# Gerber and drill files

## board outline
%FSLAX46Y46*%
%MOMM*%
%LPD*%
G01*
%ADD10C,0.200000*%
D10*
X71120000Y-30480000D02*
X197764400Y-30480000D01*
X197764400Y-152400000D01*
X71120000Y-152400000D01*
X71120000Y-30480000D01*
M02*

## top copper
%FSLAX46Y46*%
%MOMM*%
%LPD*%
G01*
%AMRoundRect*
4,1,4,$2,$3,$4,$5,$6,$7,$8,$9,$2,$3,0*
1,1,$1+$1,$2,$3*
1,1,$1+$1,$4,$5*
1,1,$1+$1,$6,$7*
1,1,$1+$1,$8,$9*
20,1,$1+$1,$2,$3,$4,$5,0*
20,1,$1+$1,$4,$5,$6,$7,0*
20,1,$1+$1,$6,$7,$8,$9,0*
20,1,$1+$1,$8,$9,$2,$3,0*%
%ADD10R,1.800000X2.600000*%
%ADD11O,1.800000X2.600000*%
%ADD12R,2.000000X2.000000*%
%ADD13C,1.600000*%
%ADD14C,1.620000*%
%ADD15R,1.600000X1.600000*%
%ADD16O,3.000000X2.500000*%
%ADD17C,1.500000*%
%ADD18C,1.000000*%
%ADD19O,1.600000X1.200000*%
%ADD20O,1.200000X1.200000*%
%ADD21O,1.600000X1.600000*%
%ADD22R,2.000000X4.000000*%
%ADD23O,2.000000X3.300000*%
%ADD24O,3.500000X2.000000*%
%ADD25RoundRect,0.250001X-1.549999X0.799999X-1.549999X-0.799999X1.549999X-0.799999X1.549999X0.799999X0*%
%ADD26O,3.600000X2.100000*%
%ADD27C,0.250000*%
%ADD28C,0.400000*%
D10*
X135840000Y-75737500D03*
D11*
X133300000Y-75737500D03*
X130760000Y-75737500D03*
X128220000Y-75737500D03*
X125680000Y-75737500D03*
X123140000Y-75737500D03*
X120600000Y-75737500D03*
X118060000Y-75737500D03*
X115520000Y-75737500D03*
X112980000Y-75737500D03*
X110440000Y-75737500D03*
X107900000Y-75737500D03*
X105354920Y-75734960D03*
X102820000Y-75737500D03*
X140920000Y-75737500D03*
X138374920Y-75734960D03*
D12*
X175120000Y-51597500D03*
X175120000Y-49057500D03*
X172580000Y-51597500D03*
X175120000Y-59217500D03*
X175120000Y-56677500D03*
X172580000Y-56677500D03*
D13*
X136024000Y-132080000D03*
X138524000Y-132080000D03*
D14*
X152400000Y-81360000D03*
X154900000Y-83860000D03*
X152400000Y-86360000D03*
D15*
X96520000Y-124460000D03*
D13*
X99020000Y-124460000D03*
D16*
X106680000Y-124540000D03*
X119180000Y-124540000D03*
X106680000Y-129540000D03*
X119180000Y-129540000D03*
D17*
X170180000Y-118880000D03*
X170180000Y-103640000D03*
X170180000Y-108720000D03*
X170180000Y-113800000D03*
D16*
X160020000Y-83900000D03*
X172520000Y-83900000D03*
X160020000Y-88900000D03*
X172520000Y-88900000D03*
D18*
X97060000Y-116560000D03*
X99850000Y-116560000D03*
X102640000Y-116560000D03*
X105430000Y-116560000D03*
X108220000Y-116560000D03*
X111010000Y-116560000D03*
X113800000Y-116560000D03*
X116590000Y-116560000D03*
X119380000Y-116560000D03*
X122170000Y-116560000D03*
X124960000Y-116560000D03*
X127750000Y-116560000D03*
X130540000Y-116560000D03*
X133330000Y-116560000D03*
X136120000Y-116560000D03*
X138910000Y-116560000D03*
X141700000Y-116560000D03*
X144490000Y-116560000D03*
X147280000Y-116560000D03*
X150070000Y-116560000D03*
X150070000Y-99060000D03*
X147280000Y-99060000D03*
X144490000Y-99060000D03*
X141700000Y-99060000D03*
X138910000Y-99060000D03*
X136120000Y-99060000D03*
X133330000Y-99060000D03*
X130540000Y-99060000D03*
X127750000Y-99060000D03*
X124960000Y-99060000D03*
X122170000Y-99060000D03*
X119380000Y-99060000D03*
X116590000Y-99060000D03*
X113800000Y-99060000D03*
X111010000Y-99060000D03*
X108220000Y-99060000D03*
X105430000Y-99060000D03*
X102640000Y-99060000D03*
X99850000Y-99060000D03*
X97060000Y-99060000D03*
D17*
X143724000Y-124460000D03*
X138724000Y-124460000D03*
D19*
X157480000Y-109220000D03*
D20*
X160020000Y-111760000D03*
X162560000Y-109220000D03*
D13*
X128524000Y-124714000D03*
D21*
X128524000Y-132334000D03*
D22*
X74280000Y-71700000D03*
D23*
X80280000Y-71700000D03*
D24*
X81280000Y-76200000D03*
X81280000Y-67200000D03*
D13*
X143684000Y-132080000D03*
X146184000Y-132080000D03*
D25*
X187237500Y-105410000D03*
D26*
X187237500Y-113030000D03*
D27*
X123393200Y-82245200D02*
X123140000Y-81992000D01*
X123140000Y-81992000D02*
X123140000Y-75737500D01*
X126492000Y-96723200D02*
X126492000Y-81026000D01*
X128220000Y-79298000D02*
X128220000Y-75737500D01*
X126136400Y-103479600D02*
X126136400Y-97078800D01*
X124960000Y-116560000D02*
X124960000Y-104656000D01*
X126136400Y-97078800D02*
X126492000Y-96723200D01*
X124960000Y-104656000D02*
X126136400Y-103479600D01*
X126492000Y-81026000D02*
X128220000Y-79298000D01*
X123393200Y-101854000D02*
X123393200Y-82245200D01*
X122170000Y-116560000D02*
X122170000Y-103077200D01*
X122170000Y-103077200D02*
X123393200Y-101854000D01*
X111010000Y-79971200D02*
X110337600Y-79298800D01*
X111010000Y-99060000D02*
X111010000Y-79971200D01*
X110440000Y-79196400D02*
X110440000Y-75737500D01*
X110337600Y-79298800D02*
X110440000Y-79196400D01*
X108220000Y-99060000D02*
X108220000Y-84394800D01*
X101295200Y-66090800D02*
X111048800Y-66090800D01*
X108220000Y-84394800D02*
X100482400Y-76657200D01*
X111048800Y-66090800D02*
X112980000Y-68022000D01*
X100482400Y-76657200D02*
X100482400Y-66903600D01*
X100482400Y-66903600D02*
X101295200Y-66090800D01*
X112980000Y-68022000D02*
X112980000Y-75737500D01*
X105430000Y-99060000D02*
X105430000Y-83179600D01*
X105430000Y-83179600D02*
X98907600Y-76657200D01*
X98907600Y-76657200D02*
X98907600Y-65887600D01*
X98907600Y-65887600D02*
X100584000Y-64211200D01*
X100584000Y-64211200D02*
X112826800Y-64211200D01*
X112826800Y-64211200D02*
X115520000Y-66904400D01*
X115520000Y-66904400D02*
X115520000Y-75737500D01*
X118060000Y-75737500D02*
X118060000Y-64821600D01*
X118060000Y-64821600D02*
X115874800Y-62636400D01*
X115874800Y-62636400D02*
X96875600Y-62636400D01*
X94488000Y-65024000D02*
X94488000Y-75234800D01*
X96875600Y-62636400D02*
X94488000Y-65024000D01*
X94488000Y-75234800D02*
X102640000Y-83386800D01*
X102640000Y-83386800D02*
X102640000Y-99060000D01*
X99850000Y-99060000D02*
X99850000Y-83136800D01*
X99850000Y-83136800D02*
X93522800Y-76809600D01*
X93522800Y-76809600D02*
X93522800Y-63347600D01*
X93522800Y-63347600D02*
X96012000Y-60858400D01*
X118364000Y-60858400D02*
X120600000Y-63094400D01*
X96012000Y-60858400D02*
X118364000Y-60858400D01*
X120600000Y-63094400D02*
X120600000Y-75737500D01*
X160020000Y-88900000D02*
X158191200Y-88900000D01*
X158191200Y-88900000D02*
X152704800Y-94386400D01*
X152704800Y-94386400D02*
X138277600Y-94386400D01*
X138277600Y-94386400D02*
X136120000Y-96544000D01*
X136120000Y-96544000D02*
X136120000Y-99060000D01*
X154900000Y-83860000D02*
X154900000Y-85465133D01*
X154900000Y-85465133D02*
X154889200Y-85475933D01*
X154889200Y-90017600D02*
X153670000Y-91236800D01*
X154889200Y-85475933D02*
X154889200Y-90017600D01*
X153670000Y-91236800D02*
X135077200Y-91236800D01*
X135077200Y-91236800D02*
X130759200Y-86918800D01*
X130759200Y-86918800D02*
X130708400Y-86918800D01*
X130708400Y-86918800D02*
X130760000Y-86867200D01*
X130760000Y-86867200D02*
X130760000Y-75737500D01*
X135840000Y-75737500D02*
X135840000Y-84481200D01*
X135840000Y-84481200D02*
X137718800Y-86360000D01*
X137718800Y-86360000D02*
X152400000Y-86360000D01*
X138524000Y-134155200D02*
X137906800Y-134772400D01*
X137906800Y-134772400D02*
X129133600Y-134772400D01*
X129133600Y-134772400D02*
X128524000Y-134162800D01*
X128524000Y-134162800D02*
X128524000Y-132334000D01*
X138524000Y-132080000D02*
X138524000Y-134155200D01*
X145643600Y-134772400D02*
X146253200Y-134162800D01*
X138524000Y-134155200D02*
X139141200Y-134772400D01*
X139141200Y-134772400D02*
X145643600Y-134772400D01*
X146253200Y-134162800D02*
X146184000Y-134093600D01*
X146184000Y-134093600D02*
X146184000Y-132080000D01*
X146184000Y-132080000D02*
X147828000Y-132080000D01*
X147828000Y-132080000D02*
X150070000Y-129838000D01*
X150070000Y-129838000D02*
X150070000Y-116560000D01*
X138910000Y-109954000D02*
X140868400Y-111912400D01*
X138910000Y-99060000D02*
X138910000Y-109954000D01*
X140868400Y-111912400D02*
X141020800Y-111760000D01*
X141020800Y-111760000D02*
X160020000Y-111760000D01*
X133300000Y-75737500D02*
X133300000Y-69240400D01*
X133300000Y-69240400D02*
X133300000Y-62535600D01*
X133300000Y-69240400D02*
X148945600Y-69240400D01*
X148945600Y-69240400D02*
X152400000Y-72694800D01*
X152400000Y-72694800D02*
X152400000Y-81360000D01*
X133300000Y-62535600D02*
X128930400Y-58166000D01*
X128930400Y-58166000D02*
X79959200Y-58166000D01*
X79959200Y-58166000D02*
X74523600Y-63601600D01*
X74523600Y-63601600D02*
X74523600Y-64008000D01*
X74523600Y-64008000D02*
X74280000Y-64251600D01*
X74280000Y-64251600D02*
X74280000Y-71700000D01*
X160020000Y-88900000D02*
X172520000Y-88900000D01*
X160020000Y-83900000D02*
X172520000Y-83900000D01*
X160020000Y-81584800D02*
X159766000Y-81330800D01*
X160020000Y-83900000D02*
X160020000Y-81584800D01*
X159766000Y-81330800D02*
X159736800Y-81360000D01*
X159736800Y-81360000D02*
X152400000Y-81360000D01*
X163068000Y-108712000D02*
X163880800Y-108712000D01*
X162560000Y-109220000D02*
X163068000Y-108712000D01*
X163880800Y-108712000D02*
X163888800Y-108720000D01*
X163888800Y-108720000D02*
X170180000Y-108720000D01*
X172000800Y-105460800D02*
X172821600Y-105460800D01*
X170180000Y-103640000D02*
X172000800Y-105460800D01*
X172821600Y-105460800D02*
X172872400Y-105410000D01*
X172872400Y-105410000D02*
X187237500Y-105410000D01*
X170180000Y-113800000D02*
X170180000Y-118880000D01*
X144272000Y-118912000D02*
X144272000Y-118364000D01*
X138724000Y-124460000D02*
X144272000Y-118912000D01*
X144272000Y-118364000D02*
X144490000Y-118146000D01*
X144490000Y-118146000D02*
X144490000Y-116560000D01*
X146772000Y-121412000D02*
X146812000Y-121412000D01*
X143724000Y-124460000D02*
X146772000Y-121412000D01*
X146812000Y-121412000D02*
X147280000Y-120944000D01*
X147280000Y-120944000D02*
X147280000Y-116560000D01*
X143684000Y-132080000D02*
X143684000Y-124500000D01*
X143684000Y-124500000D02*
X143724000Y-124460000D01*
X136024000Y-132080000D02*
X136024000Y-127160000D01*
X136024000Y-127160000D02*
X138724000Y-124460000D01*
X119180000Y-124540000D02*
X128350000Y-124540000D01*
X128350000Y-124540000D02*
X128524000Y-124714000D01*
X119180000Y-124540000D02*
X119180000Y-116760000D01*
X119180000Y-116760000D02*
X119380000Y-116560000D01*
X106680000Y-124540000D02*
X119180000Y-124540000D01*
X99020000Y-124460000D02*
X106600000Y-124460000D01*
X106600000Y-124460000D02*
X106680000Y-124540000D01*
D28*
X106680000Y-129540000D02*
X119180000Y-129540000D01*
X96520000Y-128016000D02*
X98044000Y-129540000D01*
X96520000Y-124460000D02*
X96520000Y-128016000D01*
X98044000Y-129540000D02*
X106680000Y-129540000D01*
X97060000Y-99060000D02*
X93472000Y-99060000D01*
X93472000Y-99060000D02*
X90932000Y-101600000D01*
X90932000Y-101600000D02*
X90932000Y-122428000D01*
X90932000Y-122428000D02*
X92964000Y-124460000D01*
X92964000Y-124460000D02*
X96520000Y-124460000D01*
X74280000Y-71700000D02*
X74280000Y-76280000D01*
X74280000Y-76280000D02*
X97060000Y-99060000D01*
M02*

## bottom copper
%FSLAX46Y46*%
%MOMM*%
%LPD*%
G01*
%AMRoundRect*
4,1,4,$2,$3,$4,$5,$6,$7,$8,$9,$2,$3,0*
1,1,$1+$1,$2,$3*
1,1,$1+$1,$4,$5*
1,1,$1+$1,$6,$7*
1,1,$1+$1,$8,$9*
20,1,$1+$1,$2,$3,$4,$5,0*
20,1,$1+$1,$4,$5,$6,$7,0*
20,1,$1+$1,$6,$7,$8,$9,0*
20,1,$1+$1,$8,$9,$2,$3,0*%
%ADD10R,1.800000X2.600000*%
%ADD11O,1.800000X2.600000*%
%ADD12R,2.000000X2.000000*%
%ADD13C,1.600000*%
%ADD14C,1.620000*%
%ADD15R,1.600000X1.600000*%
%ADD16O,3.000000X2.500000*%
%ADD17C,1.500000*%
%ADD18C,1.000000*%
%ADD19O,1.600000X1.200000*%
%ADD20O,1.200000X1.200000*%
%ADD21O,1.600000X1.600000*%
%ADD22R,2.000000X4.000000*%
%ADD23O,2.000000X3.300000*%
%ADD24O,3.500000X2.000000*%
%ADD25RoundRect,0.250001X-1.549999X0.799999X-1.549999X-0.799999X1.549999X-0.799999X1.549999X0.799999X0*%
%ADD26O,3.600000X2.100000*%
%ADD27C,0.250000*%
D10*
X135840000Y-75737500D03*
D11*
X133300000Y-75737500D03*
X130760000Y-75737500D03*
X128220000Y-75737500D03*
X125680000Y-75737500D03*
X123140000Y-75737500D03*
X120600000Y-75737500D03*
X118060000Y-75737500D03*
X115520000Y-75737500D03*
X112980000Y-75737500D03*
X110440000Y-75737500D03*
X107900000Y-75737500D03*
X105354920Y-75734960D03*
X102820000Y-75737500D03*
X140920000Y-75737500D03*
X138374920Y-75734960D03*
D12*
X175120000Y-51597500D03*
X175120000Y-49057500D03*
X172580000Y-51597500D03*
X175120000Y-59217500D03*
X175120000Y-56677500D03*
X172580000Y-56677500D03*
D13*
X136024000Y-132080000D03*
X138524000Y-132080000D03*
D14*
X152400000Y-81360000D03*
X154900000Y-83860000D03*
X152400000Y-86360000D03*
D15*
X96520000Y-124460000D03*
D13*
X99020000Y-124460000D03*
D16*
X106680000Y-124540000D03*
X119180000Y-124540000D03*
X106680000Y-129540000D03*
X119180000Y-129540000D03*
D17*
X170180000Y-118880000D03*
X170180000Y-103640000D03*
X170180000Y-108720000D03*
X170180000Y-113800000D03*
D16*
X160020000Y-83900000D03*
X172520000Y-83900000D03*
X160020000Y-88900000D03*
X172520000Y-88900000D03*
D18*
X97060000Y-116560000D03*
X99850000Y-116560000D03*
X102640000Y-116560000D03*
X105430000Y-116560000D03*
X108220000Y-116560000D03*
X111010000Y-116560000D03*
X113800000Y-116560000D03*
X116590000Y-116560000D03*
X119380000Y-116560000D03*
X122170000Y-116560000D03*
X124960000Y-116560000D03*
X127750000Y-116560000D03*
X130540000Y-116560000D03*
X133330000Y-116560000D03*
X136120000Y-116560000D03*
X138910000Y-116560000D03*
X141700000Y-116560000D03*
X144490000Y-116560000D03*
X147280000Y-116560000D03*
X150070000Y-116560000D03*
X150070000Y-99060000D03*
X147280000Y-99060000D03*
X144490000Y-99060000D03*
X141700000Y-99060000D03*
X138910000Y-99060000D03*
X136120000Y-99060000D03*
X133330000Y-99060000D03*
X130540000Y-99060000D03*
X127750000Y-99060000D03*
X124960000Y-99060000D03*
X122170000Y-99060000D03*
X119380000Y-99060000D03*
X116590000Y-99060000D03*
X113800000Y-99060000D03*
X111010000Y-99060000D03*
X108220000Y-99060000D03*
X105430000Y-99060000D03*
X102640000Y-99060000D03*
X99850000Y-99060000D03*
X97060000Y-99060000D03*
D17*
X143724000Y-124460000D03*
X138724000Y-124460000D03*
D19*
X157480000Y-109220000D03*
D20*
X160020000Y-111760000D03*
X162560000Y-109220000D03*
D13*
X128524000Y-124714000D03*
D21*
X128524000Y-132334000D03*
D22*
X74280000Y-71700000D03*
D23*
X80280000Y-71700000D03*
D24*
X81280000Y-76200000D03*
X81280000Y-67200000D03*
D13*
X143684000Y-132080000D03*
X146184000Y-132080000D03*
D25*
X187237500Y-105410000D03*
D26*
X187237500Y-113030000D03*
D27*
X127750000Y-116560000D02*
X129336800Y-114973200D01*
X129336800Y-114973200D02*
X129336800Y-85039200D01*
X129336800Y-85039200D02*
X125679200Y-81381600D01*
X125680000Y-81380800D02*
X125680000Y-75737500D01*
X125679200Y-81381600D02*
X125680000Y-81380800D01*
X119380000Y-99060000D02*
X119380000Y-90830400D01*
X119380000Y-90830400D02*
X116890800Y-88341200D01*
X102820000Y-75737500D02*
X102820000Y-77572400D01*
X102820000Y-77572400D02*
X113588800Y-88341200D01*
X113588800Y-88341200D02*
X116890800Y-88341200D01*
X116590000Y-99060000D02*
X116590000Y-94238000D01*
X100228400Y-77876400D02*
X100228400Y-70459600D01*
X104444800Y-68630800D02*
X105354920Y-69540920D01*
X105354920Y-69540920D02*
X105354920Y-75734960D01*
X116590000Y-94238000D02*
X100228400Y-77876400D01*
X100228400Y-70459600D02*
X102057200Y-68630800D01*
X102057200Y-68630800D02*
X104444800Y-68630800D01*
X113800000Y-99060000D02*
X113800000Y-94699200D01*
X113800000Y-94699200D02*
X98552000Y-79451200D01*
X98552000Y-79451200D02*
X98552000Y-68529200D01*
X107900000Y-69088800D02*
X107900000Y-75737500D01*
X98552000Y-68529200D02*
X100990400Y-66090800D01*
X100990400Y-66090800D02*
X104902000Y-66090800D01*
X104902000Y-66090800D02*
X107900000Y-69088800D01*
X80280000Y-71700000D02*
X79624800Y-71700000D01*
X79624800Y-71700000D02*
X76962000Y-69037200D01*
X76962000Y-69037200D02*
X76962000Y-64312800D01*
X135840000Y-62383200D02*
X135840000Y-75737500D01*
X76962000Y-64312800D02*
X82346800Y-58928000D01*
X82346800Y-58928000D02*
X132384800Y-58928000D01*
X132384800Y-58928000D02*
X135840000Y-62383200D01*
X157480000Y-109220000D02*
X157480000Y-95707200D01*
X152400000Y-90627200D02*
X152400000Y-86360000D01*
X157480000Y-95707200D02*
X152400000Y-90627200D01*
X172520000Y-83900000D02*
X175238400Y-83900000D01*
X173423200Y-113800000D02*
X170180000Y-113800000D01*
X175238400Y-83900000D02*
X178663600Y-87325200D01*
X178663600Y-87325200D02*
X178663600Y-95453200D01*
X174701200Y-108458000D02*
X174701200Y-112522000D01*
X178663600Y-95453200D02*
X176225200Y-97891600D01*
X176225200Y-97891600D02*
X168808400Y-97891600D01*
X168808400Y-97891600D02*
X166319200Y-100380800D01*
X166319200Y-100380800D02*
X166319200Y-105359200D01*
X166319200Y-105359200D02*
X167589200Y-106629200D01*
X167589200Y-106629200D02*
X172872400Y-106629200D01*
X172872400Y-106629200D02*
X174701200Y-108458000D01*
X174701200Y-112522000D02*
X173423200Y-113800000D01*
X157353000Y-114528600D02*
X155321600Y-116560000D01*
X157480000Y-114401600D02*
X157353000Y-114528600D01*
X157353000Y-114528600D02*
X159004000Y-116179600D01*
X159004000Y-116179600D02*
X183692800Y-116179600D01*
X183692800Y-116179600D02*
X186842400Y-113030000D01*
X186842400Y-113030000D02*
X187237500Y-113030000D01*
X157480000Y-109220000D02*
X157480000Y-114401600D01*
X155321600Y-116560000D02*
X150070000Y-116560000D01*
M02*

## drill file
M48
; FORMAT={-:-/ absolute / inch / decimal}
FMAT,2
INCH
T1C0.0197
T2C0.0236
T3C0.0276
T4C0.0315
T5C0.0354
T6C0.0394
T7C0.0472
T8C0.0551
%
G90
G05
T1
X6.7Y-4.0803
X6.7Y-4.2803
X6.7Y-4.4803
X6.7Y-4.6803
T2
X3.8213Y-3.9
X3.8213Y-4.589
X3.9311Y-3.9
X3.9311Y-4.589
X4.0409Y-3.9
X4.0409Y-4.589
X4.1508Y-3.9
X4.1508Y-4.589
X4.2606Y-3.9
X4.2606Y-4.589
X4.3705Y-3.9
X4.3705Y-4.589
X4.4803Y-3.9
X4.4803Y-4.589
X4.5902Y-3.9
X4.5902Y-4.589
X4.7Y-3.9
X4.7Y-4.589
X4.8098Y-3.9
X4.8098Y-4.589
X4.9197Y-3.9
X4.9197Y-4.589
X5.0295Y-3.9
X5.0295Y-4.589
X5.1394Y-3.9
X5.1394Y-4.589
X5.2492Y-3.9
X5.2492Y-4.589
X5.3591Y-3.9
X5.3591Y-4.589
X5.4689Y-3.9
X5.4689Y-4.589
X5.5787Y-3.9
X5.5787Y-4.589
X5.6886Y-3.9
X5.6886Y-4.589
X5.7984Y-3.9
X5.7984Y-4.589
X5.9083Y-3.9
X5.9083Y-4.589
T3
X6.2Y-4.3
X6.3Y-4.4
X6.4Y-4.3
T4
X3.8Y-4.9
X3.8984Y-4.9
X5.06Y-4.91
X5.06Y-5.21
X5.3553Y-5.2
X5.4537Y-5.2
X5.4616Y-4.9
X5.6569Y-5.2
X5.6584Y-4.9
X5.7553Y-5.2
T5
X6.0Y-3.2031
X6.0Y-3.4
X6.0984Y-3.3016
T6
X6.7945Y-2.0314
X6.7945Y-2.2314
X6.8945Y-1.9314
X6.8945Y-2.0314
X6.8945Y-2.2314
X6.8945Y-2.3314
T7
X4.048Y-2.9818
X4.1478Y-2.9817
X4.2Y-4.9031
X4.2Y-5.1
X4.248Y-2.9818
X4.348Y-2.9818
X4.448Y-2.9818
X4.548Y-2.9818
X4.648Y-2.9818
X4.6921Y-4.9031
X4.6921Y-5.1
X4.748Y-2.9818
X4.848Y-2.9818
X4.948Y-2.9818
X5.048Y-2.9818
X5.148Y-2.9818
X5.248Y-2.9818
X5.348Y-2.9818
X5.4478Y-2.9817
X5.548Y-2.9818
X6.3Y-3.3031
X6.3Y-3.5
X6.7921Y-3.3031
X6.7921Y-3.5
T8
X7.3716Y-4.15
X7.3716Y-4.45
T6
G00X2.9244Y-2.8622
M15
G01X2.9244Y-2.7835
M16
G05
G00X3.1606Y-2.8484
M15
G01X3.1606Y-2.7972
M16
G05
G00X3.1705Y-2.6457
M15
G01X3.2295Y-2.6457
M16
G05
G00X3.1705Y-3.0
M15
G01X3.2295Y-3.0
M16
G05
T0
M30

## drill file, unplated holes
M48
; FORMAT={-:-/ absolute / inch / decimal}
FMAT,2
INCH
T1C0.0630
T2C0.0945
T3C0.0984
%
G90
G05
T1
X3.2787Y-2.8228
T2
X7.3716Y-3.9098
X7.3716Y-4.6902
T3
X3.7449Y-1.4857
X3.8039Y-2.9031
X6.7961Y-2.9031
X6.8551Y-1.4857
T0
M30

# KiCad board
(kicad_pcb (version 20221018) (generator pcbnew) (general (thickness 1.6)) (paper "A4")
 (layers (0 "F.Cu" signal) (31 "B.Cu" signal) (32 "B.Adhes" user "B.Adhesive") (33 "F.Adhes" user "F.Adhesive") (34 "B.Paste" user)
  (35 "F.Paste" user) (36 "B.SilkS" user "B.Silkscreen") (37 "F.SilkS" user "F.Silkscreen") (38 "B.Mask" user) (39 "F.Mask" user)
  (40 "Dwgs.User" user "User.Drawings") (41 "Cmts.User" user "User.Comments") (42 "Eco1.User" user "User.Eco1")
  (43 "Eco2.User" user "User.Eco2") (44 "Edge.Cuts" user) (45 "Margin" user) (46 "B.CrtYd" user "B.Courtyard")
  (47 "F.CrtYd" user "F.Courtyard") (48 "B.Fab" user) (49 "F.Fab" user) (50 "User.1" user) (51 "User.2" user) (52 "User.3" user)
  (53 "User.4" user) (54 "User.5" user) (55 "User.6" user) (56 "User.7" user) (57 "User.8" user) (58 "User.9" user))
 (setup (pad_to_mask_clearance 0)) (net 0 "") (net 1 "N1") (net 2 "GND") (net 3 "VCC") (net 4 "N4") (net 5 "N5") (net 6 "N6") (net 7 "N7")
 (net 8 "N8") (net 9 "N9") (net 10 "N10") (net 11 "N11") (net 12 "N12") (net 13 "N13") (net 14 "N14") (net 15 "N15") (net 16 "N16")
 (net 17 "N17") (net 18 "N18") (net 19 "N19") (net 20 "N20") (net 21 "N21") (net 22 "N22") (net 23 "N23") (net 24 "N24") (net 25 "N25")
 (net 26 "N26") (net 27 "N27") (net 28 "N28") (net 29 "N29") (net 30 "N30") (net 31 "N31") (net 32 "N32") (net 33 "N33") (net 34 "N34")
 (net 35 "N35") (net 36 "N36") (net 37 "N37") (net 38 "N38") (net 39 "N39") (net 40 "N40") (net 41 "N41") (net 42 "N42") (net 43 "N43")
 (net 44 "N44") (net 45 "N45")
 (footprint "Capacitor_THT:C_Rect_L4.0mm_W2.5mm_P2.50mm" (layer "F.Cu") (at 136.024 132.08)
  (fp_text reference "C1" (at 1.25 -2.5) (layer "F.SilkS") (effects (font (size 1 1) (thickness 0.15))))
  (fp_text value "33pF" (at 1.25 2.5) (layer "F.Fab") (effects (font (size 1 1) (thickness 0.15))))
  (pad "1" thru_hole circle (at 0 0) (size 1.6 1.6) (drill 0.8) (layers "*.Cu" "*.Mask") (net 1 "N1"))
  (pad "2" thru_hole circle (at 2.5 0) (size 1.6 1.6) (drill 0.8) (layers "*.Cu" "*.Mask") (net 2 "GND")))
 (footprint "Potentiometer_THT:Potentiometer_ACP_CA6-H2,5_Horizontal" (layer "F.Cu") (at 152.4 81.36)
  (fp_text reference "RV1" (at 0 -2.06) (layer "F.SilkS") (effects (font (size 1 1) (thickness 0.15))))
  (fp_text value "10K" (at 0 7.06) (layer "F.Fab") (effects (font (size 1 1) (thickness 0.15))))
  (pad "1" thru_hole circle (at 0 0) (size 1.62 1.62) (drill 0.9) (layers "*.Cu" "*.Mask") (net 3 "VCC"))
  (pad "2" thru_hole circle (at 2.5 2.5) (size 1.62 1.62) (drill 0.9) (layers "*.Cu" "*.Mask") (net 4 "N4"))
  (pad "3" thru_hole circle (at 0 5) (size 1.62 1.62) (drill 0.9) (layers "*.Cu" "*.Mask") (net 2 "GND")))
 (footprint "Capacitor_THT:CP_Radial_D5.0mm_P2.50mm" (layer "F.Cu") (at 96.52 124.46)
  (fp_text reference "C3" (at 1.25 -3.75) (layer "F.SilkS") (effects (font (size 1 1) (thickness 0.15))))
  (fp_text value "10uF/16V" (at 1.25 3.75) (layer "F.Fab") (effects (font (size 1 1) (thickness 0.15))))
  (pad "1" thru_hole rect (at 0 0) (size 1.6 1.6) (drill 0.8) (layers "*.Cu" "*.Mask") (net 3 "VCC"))
  (pad "2" thru_hole circle (at 2.5 0) (size 1.6 1.6) (drill 0.8) (layers "*.Cu" "*.Mask") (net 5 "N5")))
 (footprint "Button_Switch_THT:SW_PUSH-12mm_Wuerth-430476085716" (layer "F.Cu") (at 106.68 124.54)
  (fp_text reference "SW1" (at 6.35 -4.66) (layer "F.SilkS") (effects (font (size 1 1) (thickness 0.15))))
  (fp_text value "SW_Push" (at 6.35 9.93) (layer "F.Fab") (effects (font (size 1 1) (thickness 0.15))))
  (pad "1" thru_hole oval (at 0 0) (size 3 2.5) (drill 1.2) (layers "*.Cu" "*.Mask") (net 5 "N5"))
  (pad "1" thru_hole oval (at 12.5 0) (size 3 2.5) (drill 1.2) (layers "*.Cu" "*.Mask") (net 5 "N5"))
  (pad "2" thru_hole oval (at 0 5) (size 3 2.5) (drill 1.2) (layers "*.Cu" "*.Mask") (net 3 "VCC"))
  (pad "2" thru_hole oval (at 12.5 5) (size 3 2.5) (drill 1.2) (layers "*.Cu" "*.Mask") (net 3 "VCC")))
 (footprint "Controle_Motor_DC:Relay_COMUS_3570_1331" (layer "F.Cu") (at 170.16 111.74 90)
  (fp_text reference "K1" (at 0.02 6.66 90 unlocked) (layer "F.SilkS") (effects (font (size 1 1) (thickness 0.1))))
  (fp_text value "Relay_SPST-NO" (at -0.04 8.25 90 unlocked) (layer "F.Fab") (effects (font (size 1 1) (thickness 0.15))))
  (pad "13" thru_hole circle (at -7.14 0.02 90) (size 1.5 1.5) (drill 0.5) (layers "*.Cu" "*.Mask") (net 3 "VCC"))
  (pad "14" thru_hole circle (at 8.1 0.02 90) (size 1.5 1.5) (drill 0.5) (layers "*.Cu" "*.Mask") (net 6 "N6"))
  (pad "A1" thru_hole circle (at 3.02 0.02 90) (size 1.5 1.5) (drill 0.5) (layers "*.Cu" "*.Mask") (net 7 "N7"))
  (pad "A2" thru_hole circle (at -2.06 0.02 90) (size 1.5 1.5) (drill 0.5) (layers "*.Cu" "*.Mask") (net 3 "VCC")))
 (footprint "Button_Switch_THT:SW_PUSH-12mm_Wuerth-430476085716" (layer "F.Cu") (at 160.02 83.9)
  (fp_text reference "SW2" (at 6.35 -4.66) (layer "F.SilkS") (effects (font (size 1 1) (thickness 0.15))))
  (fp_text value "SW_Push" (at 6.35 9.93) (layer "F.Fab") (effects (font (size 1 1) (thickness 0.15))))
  (pad "1" thru_hole oval (at 0 0) (size 3 2.5) (drill 1.2) (layers "*.Cu" "*.Mask") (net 3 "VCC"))
  (pad "1" thru_hole oval (at 12.5 0) (size 3 2.5) (drill 1.2) (layers "*.Cu" "*.Mask") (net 3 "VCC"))
  (pad "2" thru_hole oval (at 0 5) (size 3 2.5) (drill 1.2) (layers "*.Cu" "*.Mask") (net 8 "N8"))
  (pad "2" thru_hole oval (at 12.5 5) (size 3 2.5) (drill 1.2) (layers "*.Cu" "*.Mask") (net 8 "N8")))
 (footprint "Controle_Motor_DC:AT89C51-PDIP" (layer "F.Cu") (at 97.06 116.56)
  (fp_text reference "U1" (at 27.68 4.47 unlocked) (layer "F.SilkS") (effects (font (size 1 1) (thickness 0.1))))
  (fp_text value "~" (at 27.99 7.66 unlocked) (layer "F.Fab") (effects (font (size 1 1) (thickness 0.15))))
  (pad "1" thru_hole circle (at 0 0) (size 1 1) (drill 0.6) (layers "*.Cu" "*.Mask") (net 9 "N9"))
  (pad "2" thru_hole circle (at 2.79 0) (size 1 1) (drill 0.6) (layers "*.Cu" "*.Mask") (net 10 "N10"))
  (pad "3" thru_hole circle (at 5.58 0) (size 1 1) (drill 0.6) (layers "*.Cu" "*.Mask") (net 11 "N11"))
  (pad "4" thru_hole circle (at 8.37 0) (size 1 1) (drill 0.6) (layers "*.Cu" "*.Mask") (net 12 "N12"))
  (pad "5" thru_hole circle (at 11.16 0) (size 1 1) (drill 0.6) (layers "*.Cu" "*.Mask") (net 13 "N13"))
  (pad "6" thru_hole circle (at 13.95 0) (size 1 1) (drill 0.6) (layers "*.Cu" "*.Mask") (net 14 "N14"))
  (pad "7" thru_hole circle (at 16.74 0) (size 1 1) (drill 0.6) (layers "*.Cu" "*.Mask") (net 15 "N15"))
  (pad "8" thru_hole circle (at 19.53 0) (size 1 1) (drill 0.6) (layers "*.Cu" "*.Mask") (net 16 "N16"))
  (pad "9" thru_hole circle (at 22.32 0) (size 1 1) (drill 0.6) (layers "*.Cu" "*.Mask") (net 5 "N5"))
  (pad "10" thru_hole circle (at 25.11 0) (size 1 1) (drill 0.6) (layers "*.Cu" "*.Mask") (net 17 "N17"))
  (pad "11" thru_hole circle (at 27.9 0) (size 1 1) (drill 0.6) (layers "*.Cu" "*.Mask") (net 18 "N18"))
  (pad "12" thru_hole circle (at 30.69 0) (size 1 1) (drill 0.6) (layers "*.Cu" "*.Mask") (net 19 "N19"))
  (pad "13" thru_hole circle (at 33.48 0) (size 1 1) (drill 0.6) (layers "*.Cu" "*.Mask") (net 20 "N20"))
  (pad "14" thru_hole circle (at 36.27 0) (size 1 1) (drill 0.6) (layers "*.Cu" "*.Mask") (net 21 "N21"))
  (pad "15" thru_hole circle (at 39.06 0) (size 1 1) (drill 0.6) (layers "*.Cu" "*.Mask") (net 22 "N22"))
  (pad "16" thru_hole circle (at 41.85 0) (size 1 1) (drill 0.6) (layers "*.Cu" "*.Mask") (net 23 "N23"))
  (pad "17" thru_hole circle (at 44.64 0) (size 1 1) (drill 0.6) (layers "*.Cu" "*.Mask") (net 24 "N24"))
  (pad "18" thru_hole circle (at 47.43 0) (size 1 1) (drill 0.6) (layers "*.Cu" "*.Mask") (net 1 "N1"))
  (pad "19" thru_hole circle (at 50.22 0) (size 1 1) (drill 0.6) (layers "*.Cu" "*.Mask") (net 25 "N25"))
  (pad "20" thru_hole circle (at 53.01 0) (size 1 1) (drill 0.6) (layers "*.Cu" "*.Mask") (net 2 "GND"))
  (pad "21" thru_hole circle (at 53.01 -17.5) (size 1 1) (drill 0.6) (layers "*.Cu" "*.Mask") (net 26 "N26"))
  (pad "22" thru_hole circle (at 50.22 -17.5) (size 1 1) (drill 0.6) (layers "*.Cu" "*.Mask") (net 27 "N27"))
  (pad "23" thru_hole circle (at 47.43 -17.5) (size 1 1) (drill 0.6) (layers "*.Cu" "*.Mask") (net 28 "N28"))
  (pad "24" thru_hole circle (at 44.64 -17.5) (size 1 1) (drill 0.6) (layers "*.Cu" "*.Mask") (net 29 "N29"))
  (pad "25" thru_hole circle (at 41.85 -17.5) (size 1 1) (drill 0.6) (layers "*.Cu" "*.Mask") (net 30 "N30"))
  (pad "26" thru_hole circle (at 39.06 -17.5) (size 1 1) (drill 0.6) (layers "*.Cu" "*.Mask") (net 8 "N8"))
  (pad "27" thru_hole circle (at 36.27 -17.5) (size 1 1) (drill 0.6) (layers "*.Cu" "*.Mask") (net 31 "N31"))
  (pad "28" thru_hole circle (at 33.48 -17.5) (size 1 1) (drill 0.6) (layers "*.Cu" "*.Mask") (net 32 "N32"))
  (pad "29" thru_hole circle (at 30.69 -17.5) (size 1 1) (drill 0.6) (layers "*.Cu" "*.Mask") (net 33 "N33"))
  (pad "30" thru_hole circle (at 27.9 -17.5) (size 1 1) (drill 0.6) (layers "*.Cu" "*.Mask") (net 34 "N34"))
  (pad "31" thru_hole circle (at 25.11 -17.5) (size 1 1) (drill 0.6) (layers "*.Cu" "*.Mask") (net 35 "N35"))
  (pad "32" thru_hole circle (at 22.32 -17.5) (size 1 1) (drill 0.6) (layers "*.Cu" "*.Mask") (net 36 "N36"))
  (pad "33" thru_hole circle (at 19.53 -17.5) (size 1 1) (drill 0.6) (layers "*.Cu" "*.Mask") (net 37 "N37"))
  (pad "34" thru_hole circle (at 16.74 -17.5) (size 1 1) (drill 0.6) (layers "*.Cu" "*.Mask") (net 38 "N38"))
  (pad "35" thru_hole circle (at 13.95 -17.5) (size 1 1) (drill 0.6) (layers "*.Cu" "*.Mask") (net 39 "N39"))
  (pad "36" thru_hole circle (at 11.16 -17.5) (size 1 1) (drill 0.6) (layers "*.Cu" "*.Mask") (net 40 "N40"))
  (pad "37" thru_hole circle (at 8.37 -17.5) (size 1 1) (drill 0.6) (layers "*.Cu" "*.Mask") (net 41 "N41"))
  (pad "38" thru_hole circle (at 5.58 -17.5) (size 1 1) (drill 0.6) (layers "*.Cu" "*.Mask") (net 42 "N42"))
  (pad "39" thru_hole circle (at 2.79 -17.5) (size 1 1) (drill 0.6) (layers "*.Cu" "*.Mask") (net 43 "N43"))
  (pad "40" thru_hole circle (at 0 -17.5) (size 1 1) (drill 0.6) (layers "*.Cu" "*.Mask") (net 3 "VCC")))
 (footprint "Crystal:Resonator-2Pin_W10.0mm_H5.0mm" (layer "F.Cu") (at 143.724 124.46 180)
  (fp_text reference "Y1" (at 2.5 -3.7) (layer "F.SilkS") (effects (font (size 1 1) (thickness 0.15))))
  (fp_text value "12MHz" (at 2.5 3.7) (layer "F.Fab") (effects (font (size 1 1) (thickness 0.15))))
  (pad "1" thru_hole circle (at 0 0 180) (size 1.5 1.5) (drill 0.8) (layers "*.Cu" "*.Mask") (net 25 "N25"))
  (pad "2" thru_hole circle (at 5 0 180) (size 1.5 1.5) (drill 0.8) (layers "*.Cu" "*.Mask") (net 1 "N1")))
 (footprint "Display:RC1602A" (layer "F.Cu") (at 135.84 75.7375 180)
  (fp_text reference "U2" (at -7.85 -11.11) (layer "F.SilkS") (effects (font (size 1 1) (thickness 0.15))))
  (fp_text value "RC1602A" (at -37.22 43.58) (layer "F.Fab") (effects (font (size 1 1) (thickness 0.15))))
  (pad "" np_thru_hole circle (at -38.28 38) (size 2.5 2.5) (drill 2.5) (layers "*.Cu" "*.Mask"))
  (pad "" np_thru_hole circle (at -36.78 2) (size 2.5 2.5) (drill 2.5) (layers "*.Cu" "*.Mask"))
  (pad "" np_thru_hole circle (at 39.22 2) (size 2.5 2.5) (drill 2.5) (layers "*.Cu" "*.Mask"))
  (pad "" np_thru_hole circle (at 40.72 38) (size 2.5 2.5) (drill 2.5) (layers "*.Cu" "*.Mask"))
  (pad "1" thru_hole rect (at 0 0) (size 1.8 2.6) (drill 1.2) (layers "*.Cu" "*.Mask") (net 2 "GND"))
  (pad "2" thru_hole oval (at 2.54 0) (size 1.8 2.6) (drill 1.2) (layers "*.Cu" "*.Mask") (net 3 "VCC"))
  (pad "3" thru_hole oval (at 5.08 0) (size 1.8 2.6) (drill 1.2) (layers "*.Cu" "*.Mask") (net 4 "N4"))
  (pad "4" thru_hole oval (at 7.62 0) (size 1.8 2.6) (drill 1.2) (layers "*.Cu" "*.Mask") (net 18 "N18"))
  (pad "5" thru_hole oval (at 10.16 0) (size 1.8 2.6) (drill 1.2) (layers "*.Cu" "*.Mask") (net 19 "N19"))
  (pad "6" thru_hole oval (at 12.7 0) (size 1.8 2.6) (drill 1.2) (layers "*.Cu" "*.Mask") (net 17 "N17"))
  (pad "7" thru_hole oval (at 15.24 0) (size 1.8 2.6) (drill 1.2) (layers "*.Cu" "*.Mask") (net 43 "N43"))
  (pad "8" thru_hole oval (at 17.78 0) (size 1.8 2.6) (drill 1.2) (layers "*.Cu" "*.Mask") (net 42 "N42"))
  (pad "9" thru_hole oval (at 20.32 0) (size 1.8 2.6) (drill 1.2) (layers "*.Cu" "*.Mask") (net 41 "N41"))
  (pad "10" thru_hole oval (at 22.86 0) (size 1.8 2.6) (drill 1.2) (layers "*.Cu" "*.Mask") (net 40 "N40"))
  (pad "11" thru_hole oval (at 25.4 0) (size 1.8 2.6) (drill 1.2) (layers "*.Cu" "*.Mask") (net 39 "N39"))
  (pad "12" thru_hole oval (at 27.94 0) (size 1.8 2.6) (drill 1.2) (layers "*.Cu" "*.Mask") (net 38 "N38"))
  (pad "13" thru_hole oval (at 30.48508 0.00254) (size 1.8 2.6) (drill 1.2) (layers "*.Cu" "*.Mask") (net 37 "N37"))
  (pad "14" thru_hole oval (at 33.02 0) (size 1.8 2.6) (drill 1.2) (layers "*.Cu" "*.Mask") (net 36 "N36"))
  (pad "15" thru_hole oval (at -5.08 0) (size 1.8 2.6) (drill 1.2) (layers "*.Cu" "*.Mask") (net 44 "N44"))
  (pad "16" thru_hole oval (at -2.53492 0.00254) (size 1.8 2.6) (drill 1.2) (layers "*.Cu" "*.Mask") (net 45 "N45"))
  (pad "A1" thru_hole rect (at -39.28 24.14) (size 2 2) (drill 1) (layers "*.Cu" "*.Mask"))
  (pad "A1" thru_hole rect (at -39.28 26.68) (size 2 2) (drill 1) (layers "*.Cu" "*.Mask"))
  (pad "A1" thru_hole rect (at -36.74 24.14) (size 2 2) (drill 1) (layers "*.Cu" "*.Mask"))
  (pad "K1" thru_hole rect (at -39.28 16.52) (size 2 2) (drill 1) (layers "*.Cu" "*.Mask"))
  (pad "K1" thru_hole rect (at -39.28 19.06) (size 2 2) (drill 1) (layers "*.Cu" "*.Mask"))
  (pad "K1" thru_hole rect (at -36.74 19.06) (size 2 2) (drill 1) (layers "*.Cu" "*.Mask")))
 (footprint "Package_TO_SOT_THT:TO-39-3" (layer "F.Cu") (at 157.48 109.22)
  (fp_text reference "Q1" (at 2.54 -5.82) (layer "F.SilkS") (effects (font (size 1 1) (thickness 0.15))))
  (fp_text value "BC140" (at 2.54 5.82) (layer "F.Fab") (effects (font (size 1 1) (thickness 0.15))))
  (pad "1" thru_hole oval (at 0 0) (size 1.6 1.2) (drill 0.7) (layers "*.Cu" "*.Mask") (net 2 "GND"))
  (pad "2" thru_hole oval (at 2.54 2.54) (size 1.2 1.2) (drill 0.7) (layers "*.Cu" "*.Mask") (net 30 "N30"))
  (pad "3" thru_hole oval (at 5.08 0) (size 1.2 1.2) (drill 0.7) (layers "*.Cu" "*.Mask") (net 7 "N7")))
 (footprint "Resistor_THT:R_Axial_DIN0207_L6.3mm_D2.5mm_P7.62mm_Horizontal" (layer "F.Cu") (at 128.524 124.714 -90)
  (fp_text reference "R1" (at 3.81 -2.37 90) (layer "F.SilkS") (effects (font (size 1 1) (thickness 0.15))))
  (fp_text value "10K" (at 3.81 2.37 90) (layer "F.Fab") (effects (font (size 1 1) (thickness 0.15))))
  (pad "1" thru_hole circle (at 0 0 270) (size 1.6 1.6) (drill 0.8) (layers "*.Cu" "*.Mask") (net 5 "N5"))
  (pad "2" thru_hole oval (at 7.62 0 270) (size 1.6 1.6) (drill 0.8) (layers "*.Cu" "*.Mask") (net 2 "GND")))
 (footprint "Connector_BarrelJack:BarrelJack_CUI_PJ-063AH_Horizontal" (layer "F.Cu") (at 74.28 71.7 90)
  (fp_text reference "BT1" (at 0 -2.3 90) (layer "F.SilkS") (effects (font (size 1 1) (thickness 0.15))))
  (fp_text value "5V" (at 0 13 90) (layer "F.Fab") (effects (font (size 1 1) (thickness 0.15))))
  (pad "" np_thru_hole circle (at 0 9 90) (size 1.6 1.6) (drill 1.6) (layers "*.Cu" "*.Mask"))
  (pad "1" thru_hole rect (at 0 0 90) (size 4 2) (drill oval 3 1) (layers "*.Cu" "*.Mask") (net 3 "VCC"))
  (pad "2" thru_hole oval (at 0 6 90) (size 3.3 2) (drill oval 2.3 1) (layers "*.Cu" "*.Mask") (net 2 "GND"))
  (pad "MP" thru_hole oval (at -4.5 7 90) (size 2 3.5) (drill oval 1 2.5) (layers "*.Cu" "*.Mask"))
  (pad "MP" thru_hole oval (at 4.5 7 90) (size 2 3.5) (drill oval 1 2.5) (layers "*.Cu" "*.Mask")))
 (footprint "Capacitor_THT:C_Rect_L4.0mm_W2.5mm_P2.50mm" (layer "F.Cu") (at 143.684 132.08)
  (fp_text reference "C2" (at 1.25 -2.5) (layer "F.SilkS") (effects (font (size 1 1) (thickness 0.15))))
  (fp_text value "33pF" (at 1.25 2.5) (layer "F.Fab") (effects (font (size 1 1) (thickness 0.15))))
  (pad "1" thru_hole circle (at 0 0) (size 1.6 1.6) (drill 0.8) (layers "*.Cu" "*.Mask") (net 25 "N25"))
  (pad "2" thru_hole circle (at 2.5 0) (size 1.6 1.6) (drill 0.8) (layers "*.Cu" "*.Mask") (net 2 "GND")))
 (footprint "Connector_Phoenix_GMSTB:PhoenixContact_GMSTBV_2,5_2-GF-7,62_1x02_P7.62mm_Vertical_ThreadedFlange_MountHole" (layer "F.Cu")
  (at 187.2375 105.41 -90)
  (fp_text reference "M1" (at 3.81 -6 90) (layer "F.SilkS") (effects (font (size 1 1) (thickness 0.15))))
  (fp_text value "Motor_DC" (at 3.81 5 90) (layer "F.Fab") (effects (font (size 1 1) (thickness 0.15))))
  (pad "" np_thru_hole circle (at -6.1 0 270) (size 2.4 2.4) (drill 2.4) (layers "*.Cu" "*.Mask"))
  (pad "" np_thru_hole circle (at 13.72 0 270) (size 2.4 2.4) (drill 2.4) (layers "*.Cu" "*.Mask"))
  (pad "1" thru_hole roundrect (at 0 0 270) (size 2.1 3.6) (drill 1.4) (layers "*.Cu" "*.Mask") (roundrect_rratio 0.1190480952) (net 6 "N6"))
  (pad "2" thru_hole oval (at 7.62 0 270) (size 2.1 3.6) (drill 1.4) (layers "*.Cu" "*.Mask") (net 2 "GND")))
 (gr_rect (start 71.12 30.48) (end 197.7644 152.4) (stroke (width 0.2) (type default)) (fill none) (layer "Edge.Cuts"))
 (segment (start 136.024 132.08) (end 136.024 127.16) (width 0.25) (layer "F.Cu") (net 1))
 (segment (start 136.024 127.16) (end 138.724 124.46) (width 0.25) (layer "F.Cu") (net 1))
 (segment (start 144.49 118.146) (end 144.49 116.56) (width 0.25) (layer "F.Cu") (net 1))
 (segment (start 144.272 118.912) (end 144.272 118.364) (width 0.25) (layer "F.Cu") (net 1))
 (segment (start 144.272 118.364) (end 144.49 118.146) (width 0.25) (layer "F.Cu") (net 1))
 (segment (start 138.724 124.46) (end 144.272 118.912) (width 0.25) (layer "F.Cu") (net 1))
 (segment (start 137.7188 86.36) (end 152.4 86.36) (width 0.25) (layer "F.Cu") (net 2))
 (segment (start 135.84 75.7375) (end 135.84 84.4812) (width 0.25) (layer "F.Cu") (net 2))
 (segment (start 139.1412 134.7724) (end 145.6436 134.7724) (width 0.25) (layer "F.Cu") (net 2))
 (segment (start 137.9068 134.7724) (end 129.1336 134.7724) (width 0.25) (layer "F.Cu") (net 2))
 (segment (start 147.828 132.08) (end 150.07 129.838) (width 0.25) (layer "F.Cu") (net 2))
 (segment (start 138.524 134.1552) (end 137.9068 134.7724) (width 0.25) (layer "F.Cu") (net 2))
 (segment (start 146.184 134.0936) (end 146.184 132.08) (width 0.25) (layer "F.Cu") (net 2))
 (segment (start 145.6436 134.7724) (end 146.2532 134.1628) (width 0.25) (layer "F.Cu") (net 2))
 (segment (start 138.524 132.08) (end 138.524 134.1552) (width 0.25) (layer "F.Cu") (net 2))
 (segment (start 146.184 132.08) (end 147.828 132.08) (width 0.25) (layer "F.Cu") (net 2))
 (segment (start 135.84 84.4812) (end 137.7188 86.36) (width 0.25) (layer "F.Cu") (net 2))
 (segment (start 150.07 129.838) (end 150.07 116.56) (width 0.25) (layer "F.Cu") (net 2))
 (segment (start 146.2532 134.1628) (end 146.184 134.0936) (width 0.25) (layer "F.Cu") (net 2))
 (segment (start 128.524 134.1628) (end 128.524 132.334) (width 0.25) (layer "F.Cu") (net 2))
 (segment (start 129.1336 134.7724) (end 128.524 134.1628) (width 0.25) (layer "F.Cu") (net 2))
 (segment (start 138.524 134.1552) (end 139.1412 134.7724) (width 0.25) (layer "F.Cu") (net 2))
 (segment (start 159.004 116.1796) (end 183.6928 116.1796) (width 0.25) (layer "B.Cu") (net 2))
 (segment (start 186.8424 113.03) (end 187.2375 113.03) (width 0.25) (layer "B.Cu") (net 2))
 (segment (start 157.48 109.22) (end 157.48 95.7072) (width 0.25) (layer "B.Cu") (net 2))
 (segment (start 157.48 109.22) (end 157.48 114.4016) (width 0.25) (layer "B.Cu") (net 2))
 (segment (start 76.962 64.3128) (end 82.3468 58.928) (width 0.25) (layer "B.Cu") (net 2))
 (segment (start 79.6248 71.7) (end 76.962 69.0372) (width 0.25) (layer "B.Cu") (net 2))
 (segment (start 76.962 69.0372) (end 76.962 64.3128) (width 0.25) (layer "B.Cu") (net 2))
 (segment (start 157.48 114.4016) (end 157.353 114.5286) (width 0.25) (layer "B.Cu") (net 2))
 (segment (start 135.84 62.3832) (end 135.84 75.7375) (width 0.25) (layer "B.Cu") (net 2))
 (segment (start 183.6928 116.1796) (end 186.8424 113.03) (width 0.25) (layer "B.Cu") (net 2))
 (segment (start 152.4 90.6272) (end 152.4 86.36) (width 0.25) (layer "B.Cu") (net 2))
 (segment (start 157.353 114.5286) (end 159.004 116.1796) (width 0.25) (layer "B.Cu") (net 2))
 (segment (start 132.3848 58.928) (end 135.84 62.3832) (width 0.25) (layer "B.Cu") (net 2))
 (segment (start 157.353 114.5286) (end 155.3216 116.56) (width 0.25) (layer "B.Cu") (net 2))
 (segment (start 82.3468 58.928) (end 132.3848 58.928) (width 0.25) (layer "B.Cu") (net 2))
 (segment (start 80.28 71.7) (end 79.6248 71.7) (width 0.25) (layer "B.Cu") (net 2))
 (segment (start 155.3216 116.56) (end 150.07 116.56) (width 0.25) (layer "B.Cu") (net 2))
 (segment (start 157.48 95.7072) (end 152.4 90.6272) (width 0.25) (layer "B.Cu") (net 2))
 (segment (start 143.724 124.46) (end 146.772 121.412) (width 0.25) (layer "F.Cu") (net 25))
 (segment (start 143.684 132.08) (end 143.684 124.5) (width 0.25) (layer "F.Cu") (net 25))
 (segment (start 147.28 120.944) (end 147.28 116.56) (width 0.25) (layer "F.Cu") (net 25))
 (segment (start 143.684 124.5) (end 143.724 124.46) (width 0.25) (layer "F.Cu") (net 25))
 (segment (start 146.812 121.412) (end 147.28 120.944) (width 0.25) (layer "F.Cu") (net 25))
 (segment (start 146.772 121.412) (end 146.812 121.412) (width 0.25) (layer "F.Cu") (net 25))
 (segment (start 93.472 99.06) (end 90.932 101.6) (width 0.4) (layer "F.Cu") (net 3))
 (segment (start 160.02 83.9) (end 160.02 81.5848) (width 0.25) (layer "F.Cu") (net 3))
 (segment (start 133.3 69.2404) (end 133.3 62.5356) (width 0.25) (layer "F.Cu") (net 3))
 (segment (start 159.7368 81.36) (end 152.4 81.36) (width 0.25) (layer "F.Cu") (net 3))
 (segment (start 133.3 62.5356) (end 128.9304 58.166) (width 0.25) (layer "F.Cu") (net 3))
 (segment (start 74.28 76.28) (end 97.06 99.06) (width 0.4) (layer "F.Cu") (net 3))
 (segment (start 106.68 129.54) (end 119.18 129.54) (width 0.4) (layer "F.Cu") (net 3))
 (segment (start 148.9456 69.2404) (end 152.4 72.6948) (width 0.25) (layer "F.Cu") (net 3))
 (segment (start 159.766 81.3308) (end 159.7368 81.36) (width 0.25) (layer "F.Cu") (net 3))
 (segment (start 97.06 99.06) (end 93.472 99.06) (width 0.4) (layer "F.Cu") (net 3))
 (segment (start 96.52 128.016) (end 98.044 129.54) (width 0.4) (layer "F.Cu") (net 3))
 (segment (start 74.5236 63.6016) (end 74.5236 64.008) (width 0.25) (layer "F.Cu") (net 3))
 (segment (start 160.02 81.5848) (end 159.766 81.3308) (width 0.25) (layer "F.Cu") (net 3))
 (segment (start 79.9592 58.166) (end 74.5236 63.6016) (width 0.25) (layer "F.Cu") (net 3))
 (segment (start 133.3 75.7375) (end 133.3 69.2404) (width 0.25) (layer "F.Cu") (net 3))
 (segment (start 133.3 69.2404) (end 148.9456 69.2404) (width 0.25) (layer "F.Cu") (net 3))
 (segment (start 74.28 71.7) (end 74.28 76.28) (width 0.4) (layer "F.Cu") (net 3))
 (segment (start 90.932 101.6) (end 90.932 122.428) (width 0.4) (layer "F.Cu") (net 3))
 (segment (start 128.9304 58.166) (end 79.9592 58.166) (width 0.25) (layer "F.Cu") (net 3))
 (segment (start 170.18 113.8) (end 170.18 118.88) (width 0.25) (layer "F.Cu") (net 3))
 (segment (start 90.932 122.428) (end 92.964 124.46) (width 0.4) (layer "F.Cu") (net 3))
 (segment (start 74.5236 64.008) (end 74.28 64.2516) (width 0.25) (layer "F.Cu") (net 3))
 (segment (start 98.044 129.54) (end 106.68 129.54) (width 0.4) (layer "F.Cu") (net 3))
 (segment (start 92.964 124.46) (end 96.52 124.46) (width 0.4) (layer "F.Cu") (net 3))
 (segment (start 74.28 64.2516) (end 74.28 71.7) (width 0.25) (layer "F.Cu") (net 3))
 (segment (start 152.4 72.6948) (end 152.4 81.36) (width 0.25) (layer "F.Cu") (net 3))
 (segment (start 160.02 83.9) (end 172.52 83.9) (width 0.25) (layer "F.Cu") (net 3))
 (segment (start 96.52 124.46) (end 96.52 128.016) (width 0.4) (layer "F.Cu") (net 3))
 (segment (start 178.6636 95.4532) (end 176.2252 97.8916) (width 0.25) (layer "B.Cu") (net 3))
 (segment (start 178.6636 87.3252) (end 178.6636 95.4532) (width 0.25) (layer "B.Cu") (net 3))
 (segment (start 173.4232 113.8) (end 170.18 113.8) (width 0.25) (layer "B.Cu") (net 3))
 (segment (start 166.3192 100.3808) (end 166.3192 105.3592) (width 0.25) (layer "B.Cu") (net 3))
 (segment (start 174.7012 108.458) (end 174.7012 112.522) (width 0.25) (layer "B.Cu") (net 3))
 (segment (start 166.3192 105.3592) (end 167.5892 106.6292) (width 0.25) (layer "B.Cu") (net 3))
 (segment (start 168.8084 97.8916) (end 166.3192 100.3808) (width 0.25) (layer "B.Cu") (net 3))
 (segment (start 172.8724 106.6292) (end 174.7012 108.458) (width 0.25) (layer "B.Cu") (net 3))
 (segment (start 176.2252 97.8916) (end 168.8084 97.8916) (width 0.25) (layer "B.Cu") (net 3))
 (segment (start 167.5892 106.6292) (end 172.8724 106.6292) (width 0.25) (layer "B.Cu") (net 3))
 (segment (start 175.2384 83.9) (end 178.6636 87.3252) (width 0.25) (layer "B.Cu") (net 3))
 (segment (start 174.7012 112.522) (end 173.4232 113.8) (width 0.25) (layer "B.Cu") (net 3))
 (segment (start 172.52 83.9) (end 175.2384 83.9) (width 0.25) (layer "B.Cu") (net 3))
 (segment (start 119.18 124.54) (end 119.18 116.76) (width 0.25) (layer "F.Cu") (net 5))
 (segment (start 128.35 124.54) (end 128.524 124.714) (width 0.25) (layer "F.Cu") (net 5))
 (segment (start 119.18 124.54) (end 128.35 124.54) (width 0.25) (layer "F.Cu") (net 5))
 (segment (start 106.6 124.46) (end 106.68 124.54) (width 0.25) (layer "F.Cu") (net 5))
 (segment (start 99.02 124.46) (end 106.6 124.46) (width 0.25) (layer "F.Cu") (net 5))
 (segment (start 119.18 116.76) (end 119.38 116.56) (width 0.25) (layer "F.Cu") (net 5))
 (segment (start 106.68 124.54) (end 119.18 124.54) (width 0.25) (layer "F.Cu") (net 5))
 (segment (start 172.0008 105.4608) (end 172.8216 105.4608) (width 0.25) (layer "F.Cu") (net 6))
 (segment (start 172.8724 105.41) (end 187.2375 105.41) (width 0.25) (layer "F.Cu") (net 6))
 (segment (start 172.8216 105.4608) (end 172.8724 105.41) (width 0.25) (layer "F.Cu") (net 6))
 (segment (start 170.18 103.64) (end 172.0008 105.4608) (width 0.25) (layer "F.Cu") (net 6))
 (segment (start 163.8808 108.712) (end 163.8888 108.72) (width 0.25) (layer "F.Cu") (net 7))
 (segment (start 163.8888 108.72) (end 170.18 108.72) (width 0.25) (layer "F.Cu") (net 7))
 (segment (start 162.56 109.22) (end 163.068 108.712) (width 0.25) (layer "F.Cu") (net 7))
 (segment (start 163.068 108.712) (end 163.8808 108.712) (width 0.25) (layer "F.Cu") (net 7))
 (segment (start 138.91 109.954) (end 140.8684 111.9124) (width 0.25) (layer "F.Cu") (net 30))
 (segment (start 141.0208 111.76) (end 160.02 111.76) (width 0.25) (layer "F.Cu") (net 30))
 (segment (start 138.91 99.06) (end 138.91 109.954) (width 0.25) (layer "F.Cu") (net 30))
 (segment (start 140.8684 111.9124) (end 141.0208 111.76) (width 0.25) (layer "F.Cu") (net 30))
 (segment (start 154.9 83.86) (end 154.9 85.465133) (width 0.25) (layer "F.Cu") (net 4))
 (segment (start 130.7592 86.9188) (end 130.7084 86.9188) (width 0.25) (layer "F.Cu") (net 4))
 (segment (start 130.76 86.8672) (end 130.76 75.7375) (width 0.25) (layer "F.Cu") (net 4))
 (segment (start 154.9 85.465133) (end 154.8892 85.475933) (width 0.25) (layer "F.Cu") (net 4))
 (segment (start 153.67 91.2368) (end 135.0772 91.2368) (width 0.25) (layer "F.Cu") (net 4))
 (segment (start 130.7084 86.9188) (end 130.76 86.8672) (width 0.25) (layer "F.Cu") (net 4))
 (segment (start 154.8892 85.475933) (end 154.8892 90.0176) (width 0.25) (layer "F.Cu") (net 4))
 (segment (start 154.8892 90.0176) (end 153.67 91.2368) (width 0.25) (layer "F.Cu") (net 4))
 (segment (start 135.0772 91.2368) (end 130.7592 86.9188) (width 0.25) (layer "F.Cu") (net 4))
 (segment (start 138.2776 94.3864) (end 136.12 96.544) (width 0.25) (layer "F.Cu") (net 8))
 (segment (start 158.1912 88.9) (end 152.7048 94.3864) (width 0.25) (layer "F.Cu") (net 8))
 (segment (start 160.02 88.9) (end 172.52 88.9) (width 0.25) (layer "F.Cu") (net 8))
 (segment (start 160.02 88.9) (end 158.1912 88.9) (width 0.25) (layer "F.Cu") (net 8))
 (segment (start 136.12 96.544) (end 136.12 99.06) (width 0.25) (layer "F.Cu") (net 8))
 (segment (start 152.7048 94.3864) (end 138.2776 94.3864) (width 0.25) (layer "F.Cu") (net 8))
 (segment (start 122.17 103.0772) (end 123.3932 101.854) (width 0.25) (layer "F.Cu") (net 17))
 (segment (start 123.3932 101.854) (end 123.3932 82.2452) (width 0.25) (layer "F.Cu") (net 17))
 (segment (start 123.3932 82.2452) (end 123.14 81.992) (width 0.25) (layer "F.Cu") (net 17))
 (segment (start 123.14 81.992) (end 123.14 75.7375) (width 0.25) (layer "F.Cu") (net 17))
 (segment (start 122.17 116.56) (end 122.17 103.0772) (width 0.25) (layer "F.Cu") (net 17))
 (segment (start 128.22 79.298) (end 128.22 75.7375) (width 0.25) (layer "F.Cu") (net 18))
 (segment (start 126.492 81.026) (end 128.22 79.298) (width 0.25) (layer "F.Cu") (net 18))
 (segment (start 124.96 104.656) (end 126.1364 103.4796) (width 0.25) (layer "F.Cu") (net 18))
 (segment (start 126.492 96.7232) (end 126.492 81.026) (width 0.25) (layer "F.Cu") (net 18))
 (segment (start 126.1364 103.4796) (end 126.1364 97.0788) (width 0.25) (layer "F.Cu") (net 18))
 (segment (start 126.1364 97.0788) (end 126.492 96.7232) (width 0.25) (layer "F.Cu") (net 18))
 (segment (start 124.96 116.56) (end 124.96 104.656) (width 0.25) (layer "F.Cu") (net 18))
 (segment (start 127.75 116.56) (end 129.3368 114.9732) (width 0.25) (layer "B.Cu") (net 19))
 (segment (start 125.68 81.3808) (end 125.68 75.7375) (width 0.25) (layer "B.Cu") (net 19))
 (segment (start 129.3368 114.9732) (end 129.3368 85.0392) (width 0.25) (layer "B.Cu") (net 19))
 (segment (start 125.6792 81.3816) (end 125.68 81.3808) (width 0.25) (layer "B.Cu") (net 19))
 (segment (start 129.3368 85.0392) (end 125.6792 81.3816) (width 0.25) (layer "B.Cu") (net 19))
 (segment (start 119.38 90.8304) (end 116.8908 88.3412) (width 0.25) (layer "B.Cu") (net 36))
 (segment (start 113.5888 88.3412) (end 116.8908 88.3412) (width 0.25) (layer "B.Cu") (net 36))
 (segment (start 102.82 75.7375) (end 102.82 77.5724) (width 0.25) (layer "B.Cu") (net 36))
 (segment (start 102.82 77.5724) (end 113.5888 88.3412) (width 0.25) (layer "B.Cu") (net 36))
 (segment (start 119.38 99.06) (end 119.38 90.8304) (width 0.25) (layer "B.Cu") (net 36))
 (segment (start 116.59 99.06) (end 116.59 94.238) (width 0.25) (layer "B.Cu") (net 37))
 (segment (start 105.35492 69.54092) (end 105.35492 75.73496) (width 0.25) (layer "B.Cu") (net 37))
 (segment (start 100.2284 77.8764) (end 100.2284 70.4596) (width 0.25) (layer "B.Cu") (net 37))
 (segment (start 102.0572 68.6308) (end 104.4448 68.6308) (width 0.25) (layer "B.Cu") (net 37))
 (segment (start 100.2284 70.4596) (end 102.0572 68.6308) (width 0.25) (layer "B.Cu") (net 37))
 (segment (start 104.4448 68.6308) (end 105.35492 69.54092) (width 0.25) (layer "B.Cu") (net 37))
 (segment (start 116.59 94.238) (end 100.2284 77.8764) (width 0.25) (layer "B.Cu") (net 37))
 (segment (start 104.902 66.0908) (end 107.9 69.0888) (width 0.25) (layer "B.Cu") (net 38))
 (segment (start 107.9 69.0888) (end 107.9 75.7375) (width 0.25) (layer "B.Cu") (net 38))
 (segment (start 113.8 99.06) (end 113.8 94.6992) (width 0.25) (layer "B.Cu") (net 38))
 (segment (start 98.552 79.4512) (end 98.552 68.5292) (width 0.25) (layer "B.Cu") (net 38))
 (segment (start 98.552 68.5292) (end 100.9904 66.0908) (width 0.25) (layer "B.Cu") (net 38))
 (segment (start 113.8 94.6992) (end 98.552 79.4512) (width 0.25) (layer "B.Cu") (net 38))
 (segment (start 100.9904 66.0908) (end 104.902 66.0908) (width 0.25) (layer "B.Cu") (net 38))
 (segment (start 110.3376 79.2988) (end 110.44 79.1964) (width 0.25) (layer "F.Cu") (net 39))
 (segment (start 110.44 79.1964) (end 110.44 75.7375) (width 0.25) (layer "F.Cu") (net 39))
 (segment (start 111.01 79.9712) (end 110.3376 79.2988) (width 0.25) (layer "F.Cu") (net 39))
 (segment (start 111.01 99.06) (end 111.01 79.9712) (width 0.25) (layer "F.Cu") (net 39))
 (segment (start 112.98 68.022) (end 112.98 75.7375) (width 0.25) (layer "F.Cu") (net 40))
 (segment (start 101.2952 66.0908) (end 111.0488 66.0908) (width 0.25) (layer "F.Cu") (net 40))
 (segment (start 108.22 99.06) (end 108.22 84.3948) (width 0.25) (layer "F.Cu") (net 40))
 (segment (start 108.22 84.3948) (end 100.4824 76.6572) (width 0.25) (layer "F.Cu") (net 40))
 (segment (start 100.4824 66.9036) (end 101.2952 66.0908) (width 0.25) (layer "F.Cu") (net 40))
 (segment (start 100.4824 76.6572) (end 100.4824 66.9036) (width 0.25) (layer "F.Cu") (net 40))
 (segment (start 111.0488 66.0908) (end 112.98 68.022) (width 0.25) (layer "F.Cu") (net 40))
 (segment (start 112.8268 64.2112) (end 115.52 66.9044) (width 0.25) (layer "F.Cu") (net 41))
 (segment (start 98.9076 65.8876) (end 100.584 64.2112) (width 0.25) (layer "F.Cu") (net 41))
 (segment (start 105.43 99.06) (end 105.43 83.1796) (width 0.25) (layer "F.Cu") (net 41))
 (segment (start 115.52 66.9044) (end 115.52 75.7375) (width 0.25) (layer "F.Cu") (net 41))
 (segment (start 105.43 83.1796) (end 98.9076 76.6572) (width 0.25) (layer "F.Cu") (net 41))
 (segment (start 100.584 64.2112) (end 112.8268 64.2112) (width 0.25) (layer "F.Cu") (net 41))
 (segment (start 98.9076 76.6572) (end 98.9076 65.8876) (width 0.25) (layer "F.Cu") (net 41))
 (segment (start 118.06 64.8216) (end 115.8748 62.6364) (width 0.25) (layer "F.Cu") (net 42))
 (segment (start 115.8748 62.6364) (end 96.8756 62.6364) (width 0.25) (layer "F.Cu") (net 42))
 (segment (start 96.8756 62.6364) (end 94.488 65.024) (width 0.25) (layer "F.Cu") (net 42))
 (segment (start 118.06 75.7375) (end 118.06 64.8216) (width 0.25) (layer "F.Cu") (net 42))
 (segment (start 102.64 83.3868) (end 102.64 99.06) (width 0.25) (layer "F.Cu") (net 42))
 (segment (start 94.488 75.2348) (end 102.64 83.3868) (width 0.25) (layer "F.Cu") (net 42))
 (segment (start 94.488 65.024) (end 94.488 75.2348) (width 0.25) (layer "F.Cu") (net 42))
 (segment (start 99.85 99.06) (end 99.85 83.1368) (width 0.25) (layer "F.Cu") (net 43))
 (segment (start 118.364 60.8584) (end 120.6 63.0944) (width 0.25) (layer "F.Cu") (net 43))
 (segment (start 96.012 60.8584) (end 118.364 60.8584) (width 0.25) (layer "F.Cu") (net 43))
 (segment (start 99.85 83.1368) (end 93.5228 76.8096) (width 0.25) (layer "F.Cu") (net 43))
 (segment (start 93.5228 76.8096) (end 93.5228 63.3476) (width 0.25) (layer "F.Cu") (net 43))
 (segment (start 93.5228 63.3476) (end 96.012 60.8584) (width 0.25) (layer "F.Cu") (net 43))
 (segment (start 120.6 63.0944) (end 120.6 75.7375) (width 0.25) (layer "F.Cu") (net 43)))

